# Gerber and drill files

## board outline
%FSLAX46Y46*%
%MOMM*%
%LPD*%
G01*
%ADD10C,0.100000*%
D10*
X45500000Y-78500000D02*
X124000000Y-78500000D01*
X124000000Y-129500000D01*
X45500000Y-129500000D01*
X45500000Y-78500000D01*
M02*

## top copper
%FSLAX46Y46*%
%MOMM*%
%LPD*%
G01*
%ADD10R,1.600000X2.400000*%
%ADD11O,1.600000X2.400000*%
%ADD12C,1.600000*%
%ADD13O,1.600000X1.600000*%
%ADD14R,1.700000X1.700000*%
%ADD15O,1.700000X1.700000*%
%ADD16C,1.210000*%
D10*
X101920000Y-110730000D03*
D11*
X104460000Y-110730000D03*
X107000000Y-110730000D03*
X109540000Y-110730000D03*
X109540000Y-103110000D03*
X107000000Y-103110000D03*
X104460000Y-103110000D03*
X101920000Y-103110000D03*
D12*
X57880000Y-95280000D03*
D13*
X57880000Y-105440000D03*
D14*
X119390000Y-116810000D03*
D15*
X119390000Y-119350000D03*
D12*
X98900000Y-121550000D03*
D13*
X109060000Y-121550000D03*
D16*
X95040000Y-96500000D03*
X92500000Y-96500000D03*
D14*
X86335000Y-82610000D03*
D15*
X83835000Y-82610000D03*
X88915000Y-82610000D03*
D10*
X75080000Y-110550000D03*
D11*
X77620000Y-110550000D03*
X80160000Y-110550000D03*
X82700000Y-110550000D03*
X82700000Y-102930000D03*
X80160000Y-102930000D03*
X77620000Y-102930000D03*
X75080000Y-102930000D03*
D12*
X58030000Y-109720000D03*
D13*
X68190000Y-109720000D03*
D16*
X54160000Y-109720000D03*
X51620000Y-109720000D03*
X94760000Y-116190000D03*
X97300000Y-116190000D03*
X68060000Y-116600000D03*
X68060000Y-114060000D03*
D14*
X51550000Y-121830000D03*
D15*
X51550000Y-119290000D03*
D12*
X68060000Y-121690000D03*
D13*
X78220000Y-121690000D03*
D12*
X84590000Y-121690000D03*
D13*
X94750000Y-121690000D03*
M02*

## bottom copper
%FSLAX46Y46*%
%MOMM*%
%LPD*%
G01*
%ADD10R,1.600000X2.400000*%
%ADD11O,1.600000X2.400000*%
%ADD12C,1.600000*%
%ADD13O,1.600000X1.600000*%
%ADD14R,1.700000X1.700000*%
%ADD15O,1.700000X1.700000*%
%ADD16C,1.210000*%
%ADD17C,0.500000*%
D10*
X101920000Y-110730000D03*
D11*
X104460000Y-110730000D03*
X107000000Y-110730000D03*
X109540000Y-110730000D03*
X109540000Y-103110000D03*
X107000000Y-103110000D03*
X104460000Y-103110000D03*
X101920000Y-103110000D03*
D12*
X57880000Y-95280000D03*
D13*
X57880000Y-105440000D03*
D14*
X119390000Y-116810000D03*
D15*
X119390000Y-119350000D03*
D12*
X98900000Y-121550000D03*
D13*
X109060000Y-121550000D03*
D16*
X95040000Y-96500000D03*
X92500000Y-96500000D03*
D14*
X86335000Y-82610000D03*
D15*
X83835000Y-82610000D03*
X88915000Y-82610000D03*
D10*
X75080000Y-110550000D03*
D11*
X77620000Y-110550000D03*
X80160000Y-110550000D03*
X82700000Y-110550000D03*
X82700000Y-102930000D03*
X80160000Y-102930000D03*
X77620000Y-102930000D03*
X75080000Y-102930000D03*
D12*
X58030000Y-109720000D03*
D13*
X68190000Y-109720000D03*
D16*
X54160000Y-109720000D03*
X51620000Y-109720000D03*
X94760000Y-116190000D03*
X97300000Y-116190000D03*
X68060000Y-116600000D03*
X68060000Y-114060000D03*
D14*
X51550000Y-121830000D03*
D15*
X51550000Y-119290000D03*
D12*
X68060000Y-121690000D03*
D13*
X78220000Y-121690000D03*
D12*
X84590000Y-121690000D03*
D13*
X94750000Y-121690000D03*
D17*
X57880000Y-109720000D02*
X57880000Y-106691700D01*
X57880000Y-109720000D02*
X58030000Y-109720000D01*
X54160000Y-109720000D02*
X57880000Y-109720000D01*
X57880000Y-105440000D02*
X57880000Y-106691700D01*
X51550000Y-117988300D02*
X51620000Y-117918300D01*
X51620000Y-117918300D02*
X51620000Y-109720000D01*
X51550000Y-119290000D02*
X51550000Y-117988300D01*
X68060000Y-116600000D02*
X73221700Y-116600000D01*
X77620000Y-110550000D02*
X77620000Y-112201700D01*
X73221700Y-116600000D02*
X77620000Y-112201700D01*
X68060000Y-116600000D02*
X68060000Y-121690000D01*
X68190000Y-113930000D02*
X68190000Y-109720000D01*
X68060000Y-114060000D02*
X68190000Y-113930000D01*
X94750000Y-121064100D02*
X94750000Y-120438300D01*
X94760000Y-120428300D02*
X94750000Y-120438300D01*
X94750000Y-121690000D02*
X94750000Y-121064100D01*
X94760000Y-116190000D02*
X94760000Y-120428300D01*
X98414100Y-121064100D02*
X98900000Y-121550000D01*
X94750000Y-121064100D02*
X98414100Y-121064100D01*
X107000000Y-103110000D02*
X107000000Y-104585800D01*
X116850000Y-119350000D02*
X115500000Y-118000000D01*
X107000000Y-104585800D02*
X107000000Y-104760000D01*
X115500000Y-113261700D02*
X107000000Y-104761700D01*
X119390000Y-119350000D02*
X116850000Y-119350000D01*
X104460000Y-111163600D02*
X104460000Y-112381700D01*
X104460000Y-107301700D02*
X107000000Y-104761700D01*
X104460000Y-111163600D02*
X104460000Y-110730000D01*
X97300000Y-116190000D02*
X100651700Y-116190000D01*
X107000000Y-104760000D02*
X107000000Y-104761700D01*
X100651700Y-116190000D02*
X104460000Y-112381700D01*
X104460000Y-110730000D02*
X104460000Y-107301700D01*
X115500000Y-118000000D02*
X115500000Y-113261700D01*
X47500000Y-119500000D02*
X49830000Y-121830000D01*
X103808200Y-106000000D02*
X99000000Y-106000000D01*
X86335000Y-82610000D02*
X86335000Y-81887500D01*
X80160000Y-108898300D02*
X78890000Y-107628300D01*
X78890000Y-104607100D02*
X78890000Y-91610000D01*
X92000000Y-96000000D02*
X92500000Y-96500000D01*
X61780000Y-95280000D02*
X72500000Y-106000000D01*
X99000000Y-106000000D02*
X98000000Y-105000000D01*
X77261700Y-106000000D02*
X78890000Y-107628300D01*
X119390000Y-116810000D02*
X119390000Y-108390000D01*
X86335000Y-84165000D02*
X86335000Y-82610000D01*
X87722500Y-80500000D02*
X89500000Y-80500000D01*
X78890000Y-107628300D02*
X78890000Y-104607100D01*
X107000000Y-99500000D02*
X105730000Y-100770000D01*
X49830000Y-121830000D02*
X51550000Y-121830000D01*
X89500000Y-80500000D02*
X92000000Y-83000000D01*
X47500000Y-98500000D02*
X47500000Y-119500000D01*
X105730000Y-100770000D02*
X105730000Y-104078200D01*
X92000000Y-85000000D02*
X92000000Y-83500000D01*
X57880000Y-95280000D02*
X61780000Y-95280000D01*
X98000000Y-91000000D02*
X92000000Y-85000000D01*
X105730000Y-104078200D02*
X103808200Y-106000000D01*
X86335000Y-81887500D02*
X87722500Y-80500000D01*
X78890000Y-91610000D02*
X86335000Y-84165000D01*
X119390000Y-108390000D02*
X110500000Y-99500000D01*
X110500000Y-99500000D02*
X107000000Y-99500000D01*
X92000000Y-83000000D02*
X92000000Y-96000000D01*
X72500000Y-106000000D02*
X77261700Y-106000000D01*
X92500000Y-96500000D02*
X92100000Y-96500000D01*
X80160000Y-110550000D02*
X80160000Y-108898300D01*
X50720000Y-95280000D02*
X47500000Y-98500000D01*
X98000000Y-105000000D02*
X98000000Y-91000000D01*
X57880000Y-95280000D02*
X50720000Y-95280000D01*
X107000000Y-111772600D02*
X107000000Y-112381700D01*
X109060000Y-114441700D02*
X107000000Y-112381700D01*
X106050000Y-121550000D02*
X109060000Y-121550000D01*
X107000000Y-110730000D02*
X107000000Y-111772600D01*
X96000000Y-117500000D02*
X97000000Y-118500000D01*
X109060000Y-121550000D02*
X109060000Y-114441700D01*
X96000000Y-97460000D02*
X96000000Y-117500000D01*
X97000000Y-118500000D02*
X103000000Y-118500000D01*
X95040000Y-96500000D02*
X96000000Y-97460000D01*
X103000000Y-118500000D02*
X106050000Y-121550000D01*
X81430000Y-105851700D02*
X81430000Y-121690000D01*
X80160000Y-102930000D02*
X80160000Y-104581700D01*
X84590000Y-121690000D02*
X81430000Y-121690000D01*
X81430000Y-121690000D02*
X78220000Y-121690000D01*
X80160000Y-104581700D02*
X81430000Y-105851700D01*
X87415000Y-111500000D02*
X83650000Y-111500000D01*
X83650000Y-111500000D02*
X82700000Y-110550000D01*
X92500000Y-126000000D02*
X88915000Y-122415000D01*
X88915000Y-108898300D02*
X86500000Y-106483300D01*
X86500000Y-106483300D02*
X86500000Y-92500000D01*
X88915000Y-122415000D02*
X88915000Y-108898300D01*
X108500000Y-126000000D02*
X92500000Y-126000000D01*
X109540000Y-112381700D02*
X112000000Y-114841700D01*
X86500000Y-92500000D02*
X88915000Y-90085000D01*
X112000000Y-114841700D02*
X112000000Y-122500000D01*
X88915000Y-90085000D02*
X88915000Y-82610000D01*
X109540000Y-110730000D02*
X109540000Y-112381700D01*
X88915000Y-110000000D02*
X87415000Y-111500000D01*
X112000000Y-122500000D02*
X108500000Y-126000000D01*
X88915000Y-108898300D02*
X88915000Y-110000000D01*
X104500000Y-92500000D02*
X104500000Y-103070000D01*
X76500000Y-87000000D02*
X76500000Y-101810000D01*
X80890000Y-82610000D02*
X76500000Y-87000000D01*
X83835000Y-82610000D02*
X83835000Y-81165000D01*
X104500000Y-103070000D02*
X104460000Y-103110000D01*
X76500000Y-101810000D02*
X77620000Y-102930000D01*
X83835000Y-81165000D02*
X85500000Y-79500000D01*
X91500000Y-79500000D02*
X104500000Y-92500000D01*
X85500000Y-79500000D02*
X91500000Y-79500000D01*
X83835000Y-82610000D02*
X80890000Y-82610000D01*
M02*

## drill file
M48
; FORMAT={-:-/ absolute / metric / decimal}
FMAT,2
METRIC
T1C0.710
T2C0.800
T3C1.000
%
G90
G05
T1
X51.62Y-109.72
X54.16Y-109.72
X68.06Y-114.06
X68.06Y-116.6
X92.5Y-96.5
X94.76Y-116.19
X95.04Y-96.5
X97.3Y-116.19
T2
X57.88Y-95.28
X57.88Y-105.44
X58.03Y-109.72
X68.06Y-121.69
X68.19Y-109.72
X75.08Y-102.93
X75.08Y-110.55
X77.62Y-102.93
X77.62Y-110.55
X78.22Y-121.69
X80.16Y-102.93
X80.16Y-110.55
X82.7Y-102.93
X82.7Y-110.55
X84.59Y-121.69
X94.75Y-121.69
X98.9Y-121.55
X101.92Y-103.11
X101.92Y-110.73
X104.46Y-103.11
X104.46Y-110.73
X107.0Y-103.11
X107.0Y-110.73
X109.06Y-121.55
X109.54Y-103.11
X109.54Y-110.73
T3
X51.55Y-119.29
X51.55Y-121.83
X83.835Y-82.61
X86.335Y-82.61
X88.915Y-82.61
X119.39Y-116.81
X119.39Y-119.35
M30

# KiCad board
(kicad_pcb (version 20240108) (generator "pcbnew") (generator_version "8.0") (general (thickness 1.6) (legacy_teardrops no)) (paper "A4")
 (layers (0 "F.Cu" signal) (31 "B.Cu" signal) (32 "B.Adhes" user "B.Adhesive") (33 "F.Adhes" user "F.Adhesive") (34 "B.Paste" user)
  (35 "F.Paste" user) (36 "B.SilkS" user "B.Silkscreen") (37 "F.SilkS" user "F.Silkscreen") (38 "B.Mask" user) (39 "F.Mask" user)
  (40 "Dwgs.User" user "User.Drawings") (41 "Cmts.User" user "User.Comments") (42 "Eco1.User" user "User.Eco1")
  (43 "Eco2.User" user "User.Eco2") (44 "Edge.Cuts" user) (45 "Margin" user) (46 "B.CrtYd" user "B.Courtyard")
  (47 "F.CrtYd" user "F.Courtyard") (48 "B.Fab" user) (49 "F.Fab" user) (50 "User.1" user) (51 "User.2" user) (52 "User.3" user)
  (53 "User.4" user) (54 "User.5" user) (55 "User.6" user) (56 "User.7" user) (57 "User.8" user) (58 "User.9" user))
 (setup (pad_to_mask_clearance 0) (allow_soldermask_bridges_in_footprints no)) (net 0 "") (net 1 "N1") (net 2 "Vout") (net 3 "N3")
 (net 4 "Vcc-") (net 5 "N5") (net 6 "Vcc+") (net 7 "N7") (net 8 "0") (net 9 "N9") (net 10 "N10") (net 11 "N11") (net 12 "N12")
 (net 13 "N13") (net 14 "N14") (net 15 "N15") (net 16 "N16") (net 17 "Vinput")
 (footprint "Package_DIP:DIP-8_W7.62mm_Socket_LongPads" (layer "F.Cu") (at 101.92 110.73 90)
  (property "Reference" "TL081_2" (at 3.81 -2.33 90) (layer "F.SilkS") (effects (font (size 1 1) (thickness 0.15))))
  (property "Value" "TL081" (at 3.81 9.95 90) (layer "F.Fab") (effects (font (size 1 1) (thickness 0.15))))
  (pad "1" thru_hole rect (at 0 0 90) (size 2.4 1.6) (drill 0.8) (layers "*.Cu" "*.Mask") (remove_unused_layers no) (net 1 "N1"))
  (pad "2" thru_hole oval (at 0 2.54 90) (size 2.4 1.6) (drill 0.8) (layers "*.Cu" "*.Mask") (remove_unused_layers no) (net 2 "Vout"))
  (pad "3" thru_hole oval (at 0 5.08 90) (size 2.4 1.6) (drill 0.8) (layers "*.Cu" "*.Mask") (remove_unused_layers no) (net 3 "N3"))
  (pad "4" thru_hole oval (at 0 7.62 90) (size 2.4 1.6) (drill 0.8) (layers "*.Cu" "*.Mask") (remove_unused_layers no) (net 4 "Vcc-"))
  (pad "5" thru_hole oval (at 7.62 7.62 90) (size 2.4 1.6) (drill 0.8) (layers "*.Cu" "*.Mask") (remove_unused_layers no) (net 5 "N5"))
  (pad "6" thru_hole oval (at 7.62 5.08 90) (size 2.4 1.6) (drill 0.8) (layers "*.Cu" "*.Mask") (remove_unused_layers no) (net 2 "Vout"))
  (pad "7" thru_hole oval (at 7.62 2.54 90) (size 2.4 1.6) (drill 0.8) (layers "*.Cu" "*.Mask") (remove_unused_layers no) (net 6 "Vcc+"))
  (pad "8" thru_hole oval (at 7.62 0 90) (size 2.4 1.6) (drill 0.8) (layers "*.Cu" "*.Mask") (remove_unused_layers no) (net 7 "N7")))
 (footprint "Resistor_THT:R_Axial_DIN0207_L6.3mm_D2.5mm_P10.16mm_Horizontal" (layer "F.Cu") (at 57.88 95.28 -90)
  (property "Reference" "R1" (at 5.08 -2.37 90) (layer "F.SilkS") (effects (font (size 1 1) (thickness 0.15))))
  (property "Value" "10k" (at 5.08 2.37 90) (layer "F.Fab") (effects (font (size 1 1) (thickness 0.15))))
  (pad "1" thru_hole circle (at 0 0 270) (size 1.6 1.6) (drill 0.8) (layers "*.Cu" "*.Mask") (remove_unused_layers no) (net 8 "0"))
  (pad "2" thru_hole oval (at 10.16 0 270) (size 1.6 1.6) (drill 0.8) (layers "*.Cu" "*.Mask") (remove_unused_layers no) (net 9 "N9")))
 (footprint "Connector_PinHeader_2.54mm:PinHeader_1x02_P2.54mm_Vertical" (layer "F.Cu") (at 119.39 116.81)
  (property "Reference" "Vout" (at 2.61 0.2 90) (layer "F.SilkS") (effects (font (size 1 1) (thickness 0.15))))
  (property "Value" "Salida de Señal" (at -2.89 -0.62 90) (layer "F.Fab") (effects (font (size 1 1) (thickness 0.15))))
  (pad "1" thru_hole rect (at 0 0) (size 1.7 1.7) (drill 1) (layers "*.Cu" "*.Mask") (remove_unused_layers no) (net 8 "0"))
  (pad "2" thru_hole oval (at 0 2.54) (size 1.7 1.7) (drill 1) (layers "*.Cu" "*.Mask") (remove_unused_layers no) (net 2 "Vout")))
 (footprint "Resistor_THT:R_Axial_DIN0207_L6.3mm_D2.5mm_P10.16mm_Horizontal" (layer "F.Cu") (at 98.9 121.55)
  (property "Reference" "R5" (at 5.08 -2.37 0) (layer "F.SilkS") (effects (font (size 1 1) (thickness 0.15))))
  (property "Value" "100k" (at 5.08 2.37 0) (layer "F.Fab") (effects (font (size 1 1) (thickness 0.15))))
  (pad "1" thru_hole circle (at 0 0) (size 1.6 1.6) (drill 0.8) (layers "*.Cu" "*.Mask") (remove_unused_layers no) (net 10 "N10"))
  (pad "2" thru_hole oval (at 10.16 0) (size 1.6 1.6) (drill 0.8) (layers "*.Cu" "*.Mask") (remove_unused_layers no) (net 3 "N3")))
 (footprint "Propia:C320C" (layer "F.Cu") (at 86.77 103.5 180)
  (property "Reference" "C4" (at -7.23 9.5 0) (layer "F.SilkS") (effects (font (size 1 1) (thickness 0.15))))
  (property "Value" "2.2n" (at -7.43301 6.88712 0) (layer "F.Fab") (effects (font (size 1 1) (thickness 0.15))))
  (pad "1" thru_hole circle (at -8.27 7 180) (size 1.21 1.21) (drill 0.71) (layers "*.Cu" "*.Mask") (remove_unused_layers no) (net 3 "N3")
   (solder_mask_margin 0.102))
  (pad "2" thru_hole circle (at -5.73 7 180) (size 1.21 1.21) (drill 0.71) (layers "*.Cu" "*.Mask") (remove_unused_layers no) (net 8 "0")
   (solder_mask_margin 0.102)))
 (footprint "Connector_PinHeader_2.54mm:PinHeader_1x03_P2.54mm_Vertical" (layer "F.Cu") (at 83.835 82.61 90)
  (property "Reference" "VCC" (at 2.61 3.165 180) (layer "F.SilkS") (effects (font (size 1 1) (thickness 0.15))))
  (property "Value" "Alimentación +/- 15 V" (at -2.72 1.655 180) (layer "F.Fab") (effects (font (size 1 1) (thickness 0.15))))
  (pad "1" thru_hole rect (at 0 2.5 90) (size 1.7 1.7) (drill 1) (layers "*.Cu" "*.Mask") (remove_unused_layers no) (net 8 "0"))
  (pad "2" thru_hole oval (at 0 0 90) (size 1.7 1.7) (drill 1) (layers "*.Cu" "*.Mask") (remove_unused_layers no) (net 6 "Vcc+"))
  (pad "3" thru_hole oval (at 0 5.08 90) (size 1.7 1.7) (drill 1) (layers "*.Cu" "*.Mask") (remove_unused_layers no) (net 4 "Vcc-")))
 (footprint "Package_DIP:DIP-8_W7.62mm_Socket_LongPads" (layer "F.Cu") (at 75.08 110.55 90)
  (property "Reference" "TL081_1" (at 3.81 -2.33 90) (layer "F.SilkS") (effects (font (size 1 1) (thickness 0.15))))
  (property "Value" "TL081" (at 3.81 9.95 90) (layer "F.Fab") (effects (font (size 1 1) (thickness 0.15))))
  (pad "1" thru_hole rect (at 0 0 90) (size 2.4 1.6) (drill 0.8) (layers "*.Cu" "*.Mask") (remove_unused_layers no) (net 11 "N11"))
  (pad "2" thru_hole oval (at 0 2.54 90) (size 2.4 1.6) (drill 0.8) (layers "*.Cu" "*.Mask") (remove_unused_layers no) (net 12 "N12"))
  (pad "3" thru_hole oval (at 0 5.08 90) (size 2.4 1.6) (drill 0.8) (layers "*.Cu" "*.Mask") (remove_unused_layers no) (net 8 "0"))
  (pad "4" thru_hole oval (at 0 7.62 90) (size 2.4 1.6) (drill 0.8) (layers "*.Cu" "*.Mask") (remove_unused_layers no) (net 4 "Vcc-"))
  (pad "5" thru_hole oval (at 7.62 7.62 90) (size 2.4 1.6) (drill 0.8) (layers "*.Cu" "*.Mask") (remove_unused_layers no) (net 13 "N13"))
  (pad "6" thru_hole oval (at 7.62 5.08 90) (size 2.4 1.6) (drill 0.8) (layers "*.Cu" "*.Mask") (remove_unused_layers no) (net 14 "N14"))
  (pad "7" thru_hole oval (at 7.62 2.54 90) (size 2.4 1.6) (drill 0.8) (layers "*.Cu" "*.Mask") (remove_unused_layers no) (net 6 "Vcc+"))
  (pad "8" thru_hole oval (at 7.62 0 90) (size 2.4 1.6) (drill 0.8) (layers "*.Cu" "*.Mask") (remove_unused_layers no) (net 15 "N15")))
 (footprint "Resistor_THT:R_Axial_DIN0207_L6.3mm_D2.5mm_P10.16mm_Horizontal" (layer "F.Cu") (at 58.03 109.72)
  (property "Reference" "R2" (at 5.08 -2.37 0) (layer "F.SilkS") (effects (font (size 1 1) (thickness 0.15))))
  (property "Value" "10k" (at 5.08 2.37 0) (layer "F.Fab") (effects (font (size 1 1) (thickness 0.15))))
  (pad "1" thru_hole circle (at 0 0) (size 1.6 1.6) (drill 0.8) (layers "*.Cu" "*.Mask") (remove_unused_layers no) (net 9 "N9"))
  (pad "2" thru_hole oval (at 10.16 0) (size 1.6 1.6) (drill 0.8) (layers "*.Cu" "*.Mask") (remove_unused_layers no) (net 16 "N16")))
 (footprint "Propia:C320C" (layer "F.Cu") (at 45.89 116.72 180)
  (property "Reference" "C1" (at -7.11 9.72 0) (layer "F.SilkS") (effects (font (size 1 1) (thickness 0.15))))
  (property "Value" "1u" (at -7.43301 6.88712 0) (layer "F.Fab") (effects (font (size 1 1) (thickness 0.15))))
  (pad "1" thru_hole circle (at -8.27 7 180) (size 1.21 1.21) (drill 0.71) (layers "*.Cu" "*.Mask") (remove_unused_layers no) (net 9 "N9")
   (solder_mask_margin 0.102))
  (pad "2" thru_hole circle (at -5.73 7 180) (size 1.21 1.21) (drill 0.71) (layers "*.Cu" "*.Mask") (remove_unused_layers no)
   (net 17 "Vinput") (solder_mask_margin 0.102)))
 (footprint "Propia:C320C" (layer "F.Cu") (at 103.03 109.19)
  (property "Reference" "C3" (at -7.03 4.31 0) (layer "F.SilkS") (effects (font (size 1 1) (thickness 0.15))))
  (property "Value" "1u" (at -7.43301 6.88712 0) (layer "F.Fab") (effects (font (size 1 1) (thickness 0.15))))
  (pad "1" thru_hole circle (at -8.27 7) (size 1.21 1.21) (drill 0.71) (layers "*.Cu" "*.Mask") (remove_unused_layers no) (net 10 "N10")
   (solder_mask_margin 0.102))
  (pad "2" thru_hole circle (at -5.73 7) (size 1.21 1.21) (drill 0.71) (layers "*.Cu" "*.Mask") (remove_unused_layers no) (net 2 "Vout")
   (solder_mask_margin 0.102)))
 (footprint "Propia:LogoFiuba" (layer "F.Cu") (at 58.411096 84.429001)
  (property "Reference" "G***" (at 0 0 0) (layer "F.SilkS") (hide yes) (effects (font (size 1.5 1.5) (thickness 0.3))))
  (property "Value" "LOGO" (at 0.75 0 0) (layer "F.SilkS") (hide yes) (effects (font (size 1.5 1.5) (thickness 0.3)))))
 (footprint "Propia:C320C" (layer "F.Cu") (at 61.06 108.33 90)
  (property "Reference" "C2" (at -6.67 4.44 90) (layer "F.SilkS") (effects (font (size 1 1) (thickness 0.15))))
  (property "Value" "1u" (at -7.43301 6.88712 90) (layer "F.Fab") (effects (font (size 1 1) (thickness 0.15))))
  (pad "1" thru_hole circle (at -8.27 7 90) (size 1.21 1.21) (drill 0.71) (layers "*.Cu" "*.Mask") (remove_unused_layers no) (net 12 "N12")
   (solder_mask_margin 0.102))
  (pad "2" thru_hole circle (at -5.73 7 90) (size 1.21 1.21) (drill 0.71) (layers "*.Cu" "*.Mask") (remove_unused_layers no) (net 16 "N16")
   (solder_mask_margin 0.102)))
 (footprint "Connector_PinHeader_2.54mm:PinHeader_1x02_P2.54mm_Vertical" (layer "F.Cu") (at 51.55 121.83 180)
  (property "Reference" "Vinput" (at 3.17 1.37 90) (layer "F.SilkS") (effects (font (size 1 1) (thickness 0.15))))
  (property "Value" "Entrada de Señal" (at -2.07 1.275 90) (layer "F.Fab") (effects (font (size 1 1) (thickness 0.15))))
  (pad "1" thru_hole rect (at 0 0 180) (size 1.7 1.7) (drill 1) (layers "*.Cu" "*.Mask") (remove_unused_layers no) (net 8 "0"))
  (pad "2" thru_hole oval (at 0 2.54 180) (size 1.7 1.7) (drill 1) (layers "*.Cu" "*.Mask") (remove_unused_layers no) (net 17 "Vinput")))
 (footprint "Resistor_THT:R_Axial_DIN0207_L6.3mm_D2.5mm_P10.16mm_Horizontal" (layer "F.Cu") (at 68.06 121.69)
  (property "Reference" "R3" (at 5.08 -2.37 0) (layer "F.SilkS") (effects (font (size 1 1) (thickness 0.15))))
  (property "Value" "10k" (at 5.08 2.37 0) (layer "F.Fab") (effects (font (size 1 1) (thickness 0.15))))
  (pad "1" thru_hole circle (at 0 0) (size 1.6 1.6) (drill 0.8) (layers "*.Cu" "*.Mask") (remove_unused_layers no) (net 12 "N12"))
  (pad "2" thru_hole oval (at 10.16 0) (size 1.6 1.6) (drill 0.8) (layers "*.Cu" "*.Mask") (remove_unused_layers no) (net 14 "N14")))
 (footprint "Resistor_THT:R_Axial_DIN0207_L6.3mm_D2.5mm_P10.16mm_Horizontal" (layer "F.Cu") (at 84.59 121.69)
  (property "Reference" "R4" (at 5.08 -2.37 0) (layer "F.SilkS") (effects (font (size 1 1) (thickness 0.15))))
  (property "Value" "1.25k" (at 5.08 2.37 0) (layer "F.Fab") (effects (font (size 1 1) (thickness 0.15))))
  (pad "1" thru_hole circle (at 0 0) (size 1.6 1.6) (drill 0.8) (layers "*.Cu" "*.Mask") (remove_unused_layers no) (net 14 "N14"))
  (pad "2" thru_hole oval (at 10.16 0) (size 1.6 1.6) (drill 0.8) (layers "*.Cu" "*.Mask") (remove_unused_layers no) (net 10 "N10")))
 (gr_rect (start 45.5 78.5) (end 124 129.5) (stroke (width 0.1) (type default)) (fill none) (layer "Edge.Cuts"))
 (segment (start 57.88 109.72) (end 57.88 106.6917) (width 0.5) (layer "B.Cu") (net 9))
 (segment (start 57.88 109.72) (end 58.03 109.72) (width 0.5) (layer "B.Cu") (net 9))
 (segment (start 54.16 109.72) (end 57.88 109.72) (width 0.5) (layer "B.Cu") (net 9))
 (segment (start 57.88 105.44) (end 57.88 106.6917) (width 0.5) (layer "B.Cu") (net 9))
 (segment (start 51.55 117.9883) (end 51.62 117.9183) (width 0.5) (layer "B.Cu") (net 17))
 (segment (start 51.62 117.9183) (end 51.62 109.72) (width 0.5) (layer "B.Cu") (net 17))
 (segment (start 51.55 119.29) (end 51.55 117.9883) (width 0.5) (layer "B.Cu") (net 17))
 (segment (start 68.06 116.6) (end 73.2217 116.6) (width 0.5) (layer "B.Cu") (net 12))
 (segment (start 77.62 110.55) (end 77.62 112.2017) (width 0.5) (layer "B.Cu") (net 12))
 (segment (start 73.2217 116.6) (end 77.62 112.2017) (width 0.5) (layer "B.Cu") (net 12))
 (segment (start 68.06 116.6) (end 68.06 121.69) (width 0.5) (layer "B.Cu") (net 12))
 (segment (start 68.19 113.93) (end 68.19 109.72) (width 0.5) (layer "B.Cu") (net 16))
 (segment (start 68.06 114.06) (end 68.19 113.93) (width 0.5) (layer "B.Cu") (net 16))
 (segment (start 94.75 121.0641) (end 94.75 120.4383) (width 0.5) (layer "B.Cu") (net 10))
 (segment (start 94.76 120.4283) (end 94.75 120.4383) (width 0.5) (layer "B.Cu") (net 10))
 (segment (start 94.75 121.69) (end 94.75 121.0641) (width 0.5) (layer "B.Cu") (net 10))
 (segment (start 94.76 116.19) (end 94.76 120.4283) (width 0.5) (layer "B.Cu") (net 10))
 (segment (start 98.4141 121.0641) (end 98.9 121.55) (width 0.5) (layer "B.Cu") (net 10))
 (segment (start 94.75 121.0641) (end 98.4141 121.0641) (width 0.5) (layer "B.Cu") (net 10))
 (segment (start 107 103.11) (end 107 104.5858) (width 0.5) (layer "B.Cu") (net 2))
 (segment (start 116.85 119.35) (end 115.5 118) (width 0.5) (layer "B.Cu") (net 2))
 (segment (start 107 104.5858) (end 107 104.76) (width 0.5) (layer "B.Cu") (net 2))
 (segment (start 115.5 113.2617) (end 107 104.7617) (width 0.5) (layer "B.Cu") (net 2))
 (segment (start 119.39 119.35) (end 116.85 119.35) (width 0.5) (layer "B.Cu") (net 2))
 (segment (start 104.46 111.1636) (end 104.46 112.3817) (width 0.5) (layer "B.Cu") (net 2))
 (segment (start 104.46 107.3017) (end 107 104.7617) (width 0.5) (layer "B.Cu") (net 2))
 (segment (start 104.46 111.1636) (end 104.46 110.73) (width 0.5) (layer "B.Cu") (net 2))
 (segment (start 97.3 116.19) (end 100.6517 116.19) (width 0.5) (layer "B.Cu") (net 2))
 (segment (start 107 104.76) (end 107 104.7617) (width 0.5) (layer "B.Cu") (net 2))
 (segment (start 100.6517 116.19) (end 104.46 112.3817) (width 0.5) (layer "B.Cu") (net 2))
 (segment (start 104.46 110.73) (end 104.46 107.3017) (width 0.5) (layer "B.Cu") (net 2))
 (segment (start 115.5 118) (end 115.5 113.2617) (width 0.5) (layer "B.Cu") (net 2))
 (segment (start 47.5 119.5) (end 49.83 121.83) (width 0.5) (layer "B.Cu") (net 8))
 (segment (start 103.8082 106) (end 99 106) (width 0.5) (layer "B.Cu") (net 8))
 (segment (start 86.335 82.61) (end 86.335 81.8875) (width 0.5) (layer "B.Cu") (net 8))
 (segment (start 80.16 108.8983) (end 78.89 107.6283) (width 0.5) (layer "B.Cu") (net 8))
 (segment (start 78.89 104.6071) (end 78.89 91.61) (width 0.5) (layer "B.Cu") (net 8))
 (segment (start 92 96) (end 92.5 96.5) (width 0.5) (layer "B.Cu") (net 8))
 (segment (start 61.78 95.28) (end 72.5 106) (width 0.5) (layer "B.Cu") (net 8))
 (segment (start 99 106) (end 98 105) (width 0.5) (layer "B.Cu") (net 8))
 (segment (start 77.2617 106) (end 78.89 107.6283) (width 0.5) (layer "B.Cu") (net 8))
 (segment (start 119.39 116.81) (end 119.39 108.39) (width 0.5) (layer "B.Cu") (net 8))
 (segment (start 86.335 84.165) (end 86.335 82.61) (width 0.5) (layer "B.Cu") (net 8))
 (segment (start 87.7225 80.5) (end 89.5 80.5) (width 0.5) (layer "B.Cu") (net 8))
 (segment (start 78.89 107.6283) (end 78.89 104.6071) (width 0.5) (layer "B.Cu") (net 8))
 (segment (start 107 99.5) (end 105.73 100.77) (width 0.5) (layer "B.Cu") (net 8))
 (segment (start 49.83 121.83) (end 51.55 121.83) (width 0.5) (layer "B.Cu") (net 8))
 (segment (start 89.5 80.5) (end 92 83) (width 0.5) (layer "B.Cu") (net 8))
 (segment (start 47.5 98.5) (end 47.5 119.5) (width 0.5) (layer "B.Cu") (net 8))
 (segment (start 105.73 100.77) (end 105.73 104.0782) (width 0.5) (layer "B.Cu") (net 8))
 (segment (start 92 85) (end 92 83.5) (width 0.5) (layer "B.Cu") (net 8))
 (segment (start 57.88 95.28) (end 61.78 95.28) (width 0.5) (layer "B.Cu") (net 8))
 (segment (start 98 91) (end 92 85) (width 0.5) (layer "B.Cu") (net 8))
 (segment (start 105.73 104.0782) (end 103.8082 106) (width 0.5) (layer "B.Cu") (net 8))
 (segment (start 86.335 81.8875) (end 87.7225 80.5) (width 0.5) (layer "B.Cu") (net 8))
 (segment (start 78.89 91.61) (end 86.335 84.165) (width 0.5) (layer "B.Cu") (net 8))
 (segment (start 119.39 108.39) (end 110.5 99.5) (width 0.5) (layer "B.Cu") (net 8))
 (segment (start 110.5 99.5) (end 107 99.5) (width 0.5) (layer "B.Cu") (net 8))
 (segment (start 92 83) (end 92 96) (width 0.5) (layer "B.Cu") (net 8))
 (segment (start 72.5 106) (end 77.2617 106) (width 0.5) (layer "B.Cu") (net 8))
 (segment (start 92.5 96.5) (end 92.1 96.5) (width 0.5) (layer "B.Cu") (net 8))
 (segment (start 80.16 110.55) (end 80.16 108.8983) (width 0.5) (layer "B.Cu") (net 8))
 (segment (start 50.72 95.28) (end 47.5 98.5) (width 0.5) (layer "B.Cu") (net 8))
 (segment (start 98 105) (end 98 91) (width 0.5) (layer "B.Cu") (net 8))
 (segment (start 57.88 95.28) (end 50.72 95.28) (width 0.5) (layer "B.Cu") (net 8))
 (segment (start 107 111.7726) (end 107 112.3817) (width 0.5) (layer "B.Cu") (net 3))
 (segment (start 109.06 114.4417) (end 107 112.3817) (width 0.5) (layer "B.Cu") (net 3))
 (segment (start 106.05 121.55) (end 109.06 121.55) (width 0.5) (layer "B.Cu") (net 3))
 (segment (start 107 110.73) (end 107 111.7726) (width 0.5) (layer "B.Cu") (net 3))
 (segment (start 96 117.5) (end 97 118.5) (width 0.5) (layer "B.Cu") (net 3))
 (segment (start 109.06 121.55) (end 109.06 114.4417) (width 0.5) (layer "B.Cu") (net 3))
 (segment (start 96 97.46) (end 96 117.5) (width 0.5) (layer "B.Cu") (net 3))
 (segment (start 97 118.5) (end 103 118.5) (width 0.5) (layer "B.Cu") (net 3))
 (segment (start 95.04 96.5) (end 96 97.46) (width 0.5) (layer "B.Cu") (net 3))
 (segment (start 103 118.5) (end 106.05 121.55) (width 0.5) (layer "B.Cu") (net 3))
 (segment (start 81.43 105.8517) (end 81.43 121.69) (width 0.5) (layer "B.Cu") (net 14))
 (segment (start 80.16 102.93) (end 80.16 104.5817) (width 0.5) (layer "B.Cu") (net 14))
 (segment (start 84.59 121.69) (end 81.43 121.69) (width 0.5) (layer "B.Cu") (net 14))
 (segment (start 81.43 121.69) (end 78.22 121.69) (width 0.5) (layer "B.Cu") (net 14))
 (segment (start 80.16 104.5817) (end 81.43 105.8517) (width 0.5) (layer "B.Cu") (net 14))
 (segment (start 87.415 111.5) (end 83.65 111.5) (width 0.5) (layer "B.Cu") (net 4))
 (segment (start 83.65 111.5) (end 82.7 110.55) (width 0.5) (layer "B.Cu") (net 4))
 (segment (start 92.5 126) (end 88.915 122.415) (width 0.5) (layer "B.Cu") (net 4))
 (segment (start 88.915 108.8983) (end 86.5 106.4833) (width 0.5) (layer "B.Cu") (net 4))
 (segment (start 86.5 106.4833) (end 86.5 92.5) (width 0.5) (layer "B.Cu") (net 4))
 (segment (start 88.915 122.415) (end 88.915 108.8983) (width 0.5) (layer "B.Cu") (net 4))
 (segment (start 108.5 126) (end 92.5 126) (width 0.5) (layer "B.Cu") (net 4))
 (segment (start 109.54 112.3817) (end 112 114.8417) (width 0.5) (layer "B.Cu") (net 4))
 (segment (start 86.5 92.5) (end 88.915 90.085) (width 0.5) (layer "B.Cu") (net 4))
 (segment (start 112 114.8417) (end 112 122.5) (width 0.5) (layer "B.Cu") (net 4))
 (segment (start 88.915 90.085) (end 88.915 82.61) (width 0.5) (layer "B.Cu") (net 4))
 (segment (start 109.54 110.73) (end 109.54 112.3817) (width 0.5) (layer "B.Cu") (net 4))
 (segment (start 88.915 110) (end 87.415 111.5) (width 0.5) (layer "B.Cu") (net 4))
 (segment (start 112 122.5) (end 108.5 126) (width 0.5) (layer "B.Cu") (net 4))
 (segment (start 88.915 108.8983) (end 88.915 110) (width 0.5) (layer "B.Cu") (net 4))
 (segment (start 104.5 92.5) (end 104.5 103.07) (width 0.5) (layer "B.Cu") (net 6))
 (segment (start 76.5 87) (end 76.5 101.81) (width 0.5) (layer "B.Cu") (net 6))
 (segment (start 80.89 82.61) (end 76.5 87) (width 0.5) (layer "B.Cu") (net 6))
 (segment (start 83.835 82.61) (end 83.835 81.165) (width 0.5) (layer "B.Cu") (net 6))
 (segment (start 104.5 103.07) (end 104.46 103.11) (width 0.5) (layer "B.Cu") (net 6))
 (segment (start 76.5 101.81) (end 77.62 102.93) (width 0.5) (layer "B.Cu") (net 6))
 (segment (start 83.835 81.165) (end 85.5 79.5) (width 0.5) (layer "B.Cu") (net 6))
 (segment (start 91.5 79.5) (end 104.5 92.5) (width 0.5) (layer "B.Cu") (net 6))
 (segment (start 85.5 79.5) (end 91.5 79.5) (width 0.5) (layer "B.Cu") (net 6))
 (segment (start 83.835 82.61) (end 80.89 82.61) (width 0.5) (layer "B.Cu") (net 6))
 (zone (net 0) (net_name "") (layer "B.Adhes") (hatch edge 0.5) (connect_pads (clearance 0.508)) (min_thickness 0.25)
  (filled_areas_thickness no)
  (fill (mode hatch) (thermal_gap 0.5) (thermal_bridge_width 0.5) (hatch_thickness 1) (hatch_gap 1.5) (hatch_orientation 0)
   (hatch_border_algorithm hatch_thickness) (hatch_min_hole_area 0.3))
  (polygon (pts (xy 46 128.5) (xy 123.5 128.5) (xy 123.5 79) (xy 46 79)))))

